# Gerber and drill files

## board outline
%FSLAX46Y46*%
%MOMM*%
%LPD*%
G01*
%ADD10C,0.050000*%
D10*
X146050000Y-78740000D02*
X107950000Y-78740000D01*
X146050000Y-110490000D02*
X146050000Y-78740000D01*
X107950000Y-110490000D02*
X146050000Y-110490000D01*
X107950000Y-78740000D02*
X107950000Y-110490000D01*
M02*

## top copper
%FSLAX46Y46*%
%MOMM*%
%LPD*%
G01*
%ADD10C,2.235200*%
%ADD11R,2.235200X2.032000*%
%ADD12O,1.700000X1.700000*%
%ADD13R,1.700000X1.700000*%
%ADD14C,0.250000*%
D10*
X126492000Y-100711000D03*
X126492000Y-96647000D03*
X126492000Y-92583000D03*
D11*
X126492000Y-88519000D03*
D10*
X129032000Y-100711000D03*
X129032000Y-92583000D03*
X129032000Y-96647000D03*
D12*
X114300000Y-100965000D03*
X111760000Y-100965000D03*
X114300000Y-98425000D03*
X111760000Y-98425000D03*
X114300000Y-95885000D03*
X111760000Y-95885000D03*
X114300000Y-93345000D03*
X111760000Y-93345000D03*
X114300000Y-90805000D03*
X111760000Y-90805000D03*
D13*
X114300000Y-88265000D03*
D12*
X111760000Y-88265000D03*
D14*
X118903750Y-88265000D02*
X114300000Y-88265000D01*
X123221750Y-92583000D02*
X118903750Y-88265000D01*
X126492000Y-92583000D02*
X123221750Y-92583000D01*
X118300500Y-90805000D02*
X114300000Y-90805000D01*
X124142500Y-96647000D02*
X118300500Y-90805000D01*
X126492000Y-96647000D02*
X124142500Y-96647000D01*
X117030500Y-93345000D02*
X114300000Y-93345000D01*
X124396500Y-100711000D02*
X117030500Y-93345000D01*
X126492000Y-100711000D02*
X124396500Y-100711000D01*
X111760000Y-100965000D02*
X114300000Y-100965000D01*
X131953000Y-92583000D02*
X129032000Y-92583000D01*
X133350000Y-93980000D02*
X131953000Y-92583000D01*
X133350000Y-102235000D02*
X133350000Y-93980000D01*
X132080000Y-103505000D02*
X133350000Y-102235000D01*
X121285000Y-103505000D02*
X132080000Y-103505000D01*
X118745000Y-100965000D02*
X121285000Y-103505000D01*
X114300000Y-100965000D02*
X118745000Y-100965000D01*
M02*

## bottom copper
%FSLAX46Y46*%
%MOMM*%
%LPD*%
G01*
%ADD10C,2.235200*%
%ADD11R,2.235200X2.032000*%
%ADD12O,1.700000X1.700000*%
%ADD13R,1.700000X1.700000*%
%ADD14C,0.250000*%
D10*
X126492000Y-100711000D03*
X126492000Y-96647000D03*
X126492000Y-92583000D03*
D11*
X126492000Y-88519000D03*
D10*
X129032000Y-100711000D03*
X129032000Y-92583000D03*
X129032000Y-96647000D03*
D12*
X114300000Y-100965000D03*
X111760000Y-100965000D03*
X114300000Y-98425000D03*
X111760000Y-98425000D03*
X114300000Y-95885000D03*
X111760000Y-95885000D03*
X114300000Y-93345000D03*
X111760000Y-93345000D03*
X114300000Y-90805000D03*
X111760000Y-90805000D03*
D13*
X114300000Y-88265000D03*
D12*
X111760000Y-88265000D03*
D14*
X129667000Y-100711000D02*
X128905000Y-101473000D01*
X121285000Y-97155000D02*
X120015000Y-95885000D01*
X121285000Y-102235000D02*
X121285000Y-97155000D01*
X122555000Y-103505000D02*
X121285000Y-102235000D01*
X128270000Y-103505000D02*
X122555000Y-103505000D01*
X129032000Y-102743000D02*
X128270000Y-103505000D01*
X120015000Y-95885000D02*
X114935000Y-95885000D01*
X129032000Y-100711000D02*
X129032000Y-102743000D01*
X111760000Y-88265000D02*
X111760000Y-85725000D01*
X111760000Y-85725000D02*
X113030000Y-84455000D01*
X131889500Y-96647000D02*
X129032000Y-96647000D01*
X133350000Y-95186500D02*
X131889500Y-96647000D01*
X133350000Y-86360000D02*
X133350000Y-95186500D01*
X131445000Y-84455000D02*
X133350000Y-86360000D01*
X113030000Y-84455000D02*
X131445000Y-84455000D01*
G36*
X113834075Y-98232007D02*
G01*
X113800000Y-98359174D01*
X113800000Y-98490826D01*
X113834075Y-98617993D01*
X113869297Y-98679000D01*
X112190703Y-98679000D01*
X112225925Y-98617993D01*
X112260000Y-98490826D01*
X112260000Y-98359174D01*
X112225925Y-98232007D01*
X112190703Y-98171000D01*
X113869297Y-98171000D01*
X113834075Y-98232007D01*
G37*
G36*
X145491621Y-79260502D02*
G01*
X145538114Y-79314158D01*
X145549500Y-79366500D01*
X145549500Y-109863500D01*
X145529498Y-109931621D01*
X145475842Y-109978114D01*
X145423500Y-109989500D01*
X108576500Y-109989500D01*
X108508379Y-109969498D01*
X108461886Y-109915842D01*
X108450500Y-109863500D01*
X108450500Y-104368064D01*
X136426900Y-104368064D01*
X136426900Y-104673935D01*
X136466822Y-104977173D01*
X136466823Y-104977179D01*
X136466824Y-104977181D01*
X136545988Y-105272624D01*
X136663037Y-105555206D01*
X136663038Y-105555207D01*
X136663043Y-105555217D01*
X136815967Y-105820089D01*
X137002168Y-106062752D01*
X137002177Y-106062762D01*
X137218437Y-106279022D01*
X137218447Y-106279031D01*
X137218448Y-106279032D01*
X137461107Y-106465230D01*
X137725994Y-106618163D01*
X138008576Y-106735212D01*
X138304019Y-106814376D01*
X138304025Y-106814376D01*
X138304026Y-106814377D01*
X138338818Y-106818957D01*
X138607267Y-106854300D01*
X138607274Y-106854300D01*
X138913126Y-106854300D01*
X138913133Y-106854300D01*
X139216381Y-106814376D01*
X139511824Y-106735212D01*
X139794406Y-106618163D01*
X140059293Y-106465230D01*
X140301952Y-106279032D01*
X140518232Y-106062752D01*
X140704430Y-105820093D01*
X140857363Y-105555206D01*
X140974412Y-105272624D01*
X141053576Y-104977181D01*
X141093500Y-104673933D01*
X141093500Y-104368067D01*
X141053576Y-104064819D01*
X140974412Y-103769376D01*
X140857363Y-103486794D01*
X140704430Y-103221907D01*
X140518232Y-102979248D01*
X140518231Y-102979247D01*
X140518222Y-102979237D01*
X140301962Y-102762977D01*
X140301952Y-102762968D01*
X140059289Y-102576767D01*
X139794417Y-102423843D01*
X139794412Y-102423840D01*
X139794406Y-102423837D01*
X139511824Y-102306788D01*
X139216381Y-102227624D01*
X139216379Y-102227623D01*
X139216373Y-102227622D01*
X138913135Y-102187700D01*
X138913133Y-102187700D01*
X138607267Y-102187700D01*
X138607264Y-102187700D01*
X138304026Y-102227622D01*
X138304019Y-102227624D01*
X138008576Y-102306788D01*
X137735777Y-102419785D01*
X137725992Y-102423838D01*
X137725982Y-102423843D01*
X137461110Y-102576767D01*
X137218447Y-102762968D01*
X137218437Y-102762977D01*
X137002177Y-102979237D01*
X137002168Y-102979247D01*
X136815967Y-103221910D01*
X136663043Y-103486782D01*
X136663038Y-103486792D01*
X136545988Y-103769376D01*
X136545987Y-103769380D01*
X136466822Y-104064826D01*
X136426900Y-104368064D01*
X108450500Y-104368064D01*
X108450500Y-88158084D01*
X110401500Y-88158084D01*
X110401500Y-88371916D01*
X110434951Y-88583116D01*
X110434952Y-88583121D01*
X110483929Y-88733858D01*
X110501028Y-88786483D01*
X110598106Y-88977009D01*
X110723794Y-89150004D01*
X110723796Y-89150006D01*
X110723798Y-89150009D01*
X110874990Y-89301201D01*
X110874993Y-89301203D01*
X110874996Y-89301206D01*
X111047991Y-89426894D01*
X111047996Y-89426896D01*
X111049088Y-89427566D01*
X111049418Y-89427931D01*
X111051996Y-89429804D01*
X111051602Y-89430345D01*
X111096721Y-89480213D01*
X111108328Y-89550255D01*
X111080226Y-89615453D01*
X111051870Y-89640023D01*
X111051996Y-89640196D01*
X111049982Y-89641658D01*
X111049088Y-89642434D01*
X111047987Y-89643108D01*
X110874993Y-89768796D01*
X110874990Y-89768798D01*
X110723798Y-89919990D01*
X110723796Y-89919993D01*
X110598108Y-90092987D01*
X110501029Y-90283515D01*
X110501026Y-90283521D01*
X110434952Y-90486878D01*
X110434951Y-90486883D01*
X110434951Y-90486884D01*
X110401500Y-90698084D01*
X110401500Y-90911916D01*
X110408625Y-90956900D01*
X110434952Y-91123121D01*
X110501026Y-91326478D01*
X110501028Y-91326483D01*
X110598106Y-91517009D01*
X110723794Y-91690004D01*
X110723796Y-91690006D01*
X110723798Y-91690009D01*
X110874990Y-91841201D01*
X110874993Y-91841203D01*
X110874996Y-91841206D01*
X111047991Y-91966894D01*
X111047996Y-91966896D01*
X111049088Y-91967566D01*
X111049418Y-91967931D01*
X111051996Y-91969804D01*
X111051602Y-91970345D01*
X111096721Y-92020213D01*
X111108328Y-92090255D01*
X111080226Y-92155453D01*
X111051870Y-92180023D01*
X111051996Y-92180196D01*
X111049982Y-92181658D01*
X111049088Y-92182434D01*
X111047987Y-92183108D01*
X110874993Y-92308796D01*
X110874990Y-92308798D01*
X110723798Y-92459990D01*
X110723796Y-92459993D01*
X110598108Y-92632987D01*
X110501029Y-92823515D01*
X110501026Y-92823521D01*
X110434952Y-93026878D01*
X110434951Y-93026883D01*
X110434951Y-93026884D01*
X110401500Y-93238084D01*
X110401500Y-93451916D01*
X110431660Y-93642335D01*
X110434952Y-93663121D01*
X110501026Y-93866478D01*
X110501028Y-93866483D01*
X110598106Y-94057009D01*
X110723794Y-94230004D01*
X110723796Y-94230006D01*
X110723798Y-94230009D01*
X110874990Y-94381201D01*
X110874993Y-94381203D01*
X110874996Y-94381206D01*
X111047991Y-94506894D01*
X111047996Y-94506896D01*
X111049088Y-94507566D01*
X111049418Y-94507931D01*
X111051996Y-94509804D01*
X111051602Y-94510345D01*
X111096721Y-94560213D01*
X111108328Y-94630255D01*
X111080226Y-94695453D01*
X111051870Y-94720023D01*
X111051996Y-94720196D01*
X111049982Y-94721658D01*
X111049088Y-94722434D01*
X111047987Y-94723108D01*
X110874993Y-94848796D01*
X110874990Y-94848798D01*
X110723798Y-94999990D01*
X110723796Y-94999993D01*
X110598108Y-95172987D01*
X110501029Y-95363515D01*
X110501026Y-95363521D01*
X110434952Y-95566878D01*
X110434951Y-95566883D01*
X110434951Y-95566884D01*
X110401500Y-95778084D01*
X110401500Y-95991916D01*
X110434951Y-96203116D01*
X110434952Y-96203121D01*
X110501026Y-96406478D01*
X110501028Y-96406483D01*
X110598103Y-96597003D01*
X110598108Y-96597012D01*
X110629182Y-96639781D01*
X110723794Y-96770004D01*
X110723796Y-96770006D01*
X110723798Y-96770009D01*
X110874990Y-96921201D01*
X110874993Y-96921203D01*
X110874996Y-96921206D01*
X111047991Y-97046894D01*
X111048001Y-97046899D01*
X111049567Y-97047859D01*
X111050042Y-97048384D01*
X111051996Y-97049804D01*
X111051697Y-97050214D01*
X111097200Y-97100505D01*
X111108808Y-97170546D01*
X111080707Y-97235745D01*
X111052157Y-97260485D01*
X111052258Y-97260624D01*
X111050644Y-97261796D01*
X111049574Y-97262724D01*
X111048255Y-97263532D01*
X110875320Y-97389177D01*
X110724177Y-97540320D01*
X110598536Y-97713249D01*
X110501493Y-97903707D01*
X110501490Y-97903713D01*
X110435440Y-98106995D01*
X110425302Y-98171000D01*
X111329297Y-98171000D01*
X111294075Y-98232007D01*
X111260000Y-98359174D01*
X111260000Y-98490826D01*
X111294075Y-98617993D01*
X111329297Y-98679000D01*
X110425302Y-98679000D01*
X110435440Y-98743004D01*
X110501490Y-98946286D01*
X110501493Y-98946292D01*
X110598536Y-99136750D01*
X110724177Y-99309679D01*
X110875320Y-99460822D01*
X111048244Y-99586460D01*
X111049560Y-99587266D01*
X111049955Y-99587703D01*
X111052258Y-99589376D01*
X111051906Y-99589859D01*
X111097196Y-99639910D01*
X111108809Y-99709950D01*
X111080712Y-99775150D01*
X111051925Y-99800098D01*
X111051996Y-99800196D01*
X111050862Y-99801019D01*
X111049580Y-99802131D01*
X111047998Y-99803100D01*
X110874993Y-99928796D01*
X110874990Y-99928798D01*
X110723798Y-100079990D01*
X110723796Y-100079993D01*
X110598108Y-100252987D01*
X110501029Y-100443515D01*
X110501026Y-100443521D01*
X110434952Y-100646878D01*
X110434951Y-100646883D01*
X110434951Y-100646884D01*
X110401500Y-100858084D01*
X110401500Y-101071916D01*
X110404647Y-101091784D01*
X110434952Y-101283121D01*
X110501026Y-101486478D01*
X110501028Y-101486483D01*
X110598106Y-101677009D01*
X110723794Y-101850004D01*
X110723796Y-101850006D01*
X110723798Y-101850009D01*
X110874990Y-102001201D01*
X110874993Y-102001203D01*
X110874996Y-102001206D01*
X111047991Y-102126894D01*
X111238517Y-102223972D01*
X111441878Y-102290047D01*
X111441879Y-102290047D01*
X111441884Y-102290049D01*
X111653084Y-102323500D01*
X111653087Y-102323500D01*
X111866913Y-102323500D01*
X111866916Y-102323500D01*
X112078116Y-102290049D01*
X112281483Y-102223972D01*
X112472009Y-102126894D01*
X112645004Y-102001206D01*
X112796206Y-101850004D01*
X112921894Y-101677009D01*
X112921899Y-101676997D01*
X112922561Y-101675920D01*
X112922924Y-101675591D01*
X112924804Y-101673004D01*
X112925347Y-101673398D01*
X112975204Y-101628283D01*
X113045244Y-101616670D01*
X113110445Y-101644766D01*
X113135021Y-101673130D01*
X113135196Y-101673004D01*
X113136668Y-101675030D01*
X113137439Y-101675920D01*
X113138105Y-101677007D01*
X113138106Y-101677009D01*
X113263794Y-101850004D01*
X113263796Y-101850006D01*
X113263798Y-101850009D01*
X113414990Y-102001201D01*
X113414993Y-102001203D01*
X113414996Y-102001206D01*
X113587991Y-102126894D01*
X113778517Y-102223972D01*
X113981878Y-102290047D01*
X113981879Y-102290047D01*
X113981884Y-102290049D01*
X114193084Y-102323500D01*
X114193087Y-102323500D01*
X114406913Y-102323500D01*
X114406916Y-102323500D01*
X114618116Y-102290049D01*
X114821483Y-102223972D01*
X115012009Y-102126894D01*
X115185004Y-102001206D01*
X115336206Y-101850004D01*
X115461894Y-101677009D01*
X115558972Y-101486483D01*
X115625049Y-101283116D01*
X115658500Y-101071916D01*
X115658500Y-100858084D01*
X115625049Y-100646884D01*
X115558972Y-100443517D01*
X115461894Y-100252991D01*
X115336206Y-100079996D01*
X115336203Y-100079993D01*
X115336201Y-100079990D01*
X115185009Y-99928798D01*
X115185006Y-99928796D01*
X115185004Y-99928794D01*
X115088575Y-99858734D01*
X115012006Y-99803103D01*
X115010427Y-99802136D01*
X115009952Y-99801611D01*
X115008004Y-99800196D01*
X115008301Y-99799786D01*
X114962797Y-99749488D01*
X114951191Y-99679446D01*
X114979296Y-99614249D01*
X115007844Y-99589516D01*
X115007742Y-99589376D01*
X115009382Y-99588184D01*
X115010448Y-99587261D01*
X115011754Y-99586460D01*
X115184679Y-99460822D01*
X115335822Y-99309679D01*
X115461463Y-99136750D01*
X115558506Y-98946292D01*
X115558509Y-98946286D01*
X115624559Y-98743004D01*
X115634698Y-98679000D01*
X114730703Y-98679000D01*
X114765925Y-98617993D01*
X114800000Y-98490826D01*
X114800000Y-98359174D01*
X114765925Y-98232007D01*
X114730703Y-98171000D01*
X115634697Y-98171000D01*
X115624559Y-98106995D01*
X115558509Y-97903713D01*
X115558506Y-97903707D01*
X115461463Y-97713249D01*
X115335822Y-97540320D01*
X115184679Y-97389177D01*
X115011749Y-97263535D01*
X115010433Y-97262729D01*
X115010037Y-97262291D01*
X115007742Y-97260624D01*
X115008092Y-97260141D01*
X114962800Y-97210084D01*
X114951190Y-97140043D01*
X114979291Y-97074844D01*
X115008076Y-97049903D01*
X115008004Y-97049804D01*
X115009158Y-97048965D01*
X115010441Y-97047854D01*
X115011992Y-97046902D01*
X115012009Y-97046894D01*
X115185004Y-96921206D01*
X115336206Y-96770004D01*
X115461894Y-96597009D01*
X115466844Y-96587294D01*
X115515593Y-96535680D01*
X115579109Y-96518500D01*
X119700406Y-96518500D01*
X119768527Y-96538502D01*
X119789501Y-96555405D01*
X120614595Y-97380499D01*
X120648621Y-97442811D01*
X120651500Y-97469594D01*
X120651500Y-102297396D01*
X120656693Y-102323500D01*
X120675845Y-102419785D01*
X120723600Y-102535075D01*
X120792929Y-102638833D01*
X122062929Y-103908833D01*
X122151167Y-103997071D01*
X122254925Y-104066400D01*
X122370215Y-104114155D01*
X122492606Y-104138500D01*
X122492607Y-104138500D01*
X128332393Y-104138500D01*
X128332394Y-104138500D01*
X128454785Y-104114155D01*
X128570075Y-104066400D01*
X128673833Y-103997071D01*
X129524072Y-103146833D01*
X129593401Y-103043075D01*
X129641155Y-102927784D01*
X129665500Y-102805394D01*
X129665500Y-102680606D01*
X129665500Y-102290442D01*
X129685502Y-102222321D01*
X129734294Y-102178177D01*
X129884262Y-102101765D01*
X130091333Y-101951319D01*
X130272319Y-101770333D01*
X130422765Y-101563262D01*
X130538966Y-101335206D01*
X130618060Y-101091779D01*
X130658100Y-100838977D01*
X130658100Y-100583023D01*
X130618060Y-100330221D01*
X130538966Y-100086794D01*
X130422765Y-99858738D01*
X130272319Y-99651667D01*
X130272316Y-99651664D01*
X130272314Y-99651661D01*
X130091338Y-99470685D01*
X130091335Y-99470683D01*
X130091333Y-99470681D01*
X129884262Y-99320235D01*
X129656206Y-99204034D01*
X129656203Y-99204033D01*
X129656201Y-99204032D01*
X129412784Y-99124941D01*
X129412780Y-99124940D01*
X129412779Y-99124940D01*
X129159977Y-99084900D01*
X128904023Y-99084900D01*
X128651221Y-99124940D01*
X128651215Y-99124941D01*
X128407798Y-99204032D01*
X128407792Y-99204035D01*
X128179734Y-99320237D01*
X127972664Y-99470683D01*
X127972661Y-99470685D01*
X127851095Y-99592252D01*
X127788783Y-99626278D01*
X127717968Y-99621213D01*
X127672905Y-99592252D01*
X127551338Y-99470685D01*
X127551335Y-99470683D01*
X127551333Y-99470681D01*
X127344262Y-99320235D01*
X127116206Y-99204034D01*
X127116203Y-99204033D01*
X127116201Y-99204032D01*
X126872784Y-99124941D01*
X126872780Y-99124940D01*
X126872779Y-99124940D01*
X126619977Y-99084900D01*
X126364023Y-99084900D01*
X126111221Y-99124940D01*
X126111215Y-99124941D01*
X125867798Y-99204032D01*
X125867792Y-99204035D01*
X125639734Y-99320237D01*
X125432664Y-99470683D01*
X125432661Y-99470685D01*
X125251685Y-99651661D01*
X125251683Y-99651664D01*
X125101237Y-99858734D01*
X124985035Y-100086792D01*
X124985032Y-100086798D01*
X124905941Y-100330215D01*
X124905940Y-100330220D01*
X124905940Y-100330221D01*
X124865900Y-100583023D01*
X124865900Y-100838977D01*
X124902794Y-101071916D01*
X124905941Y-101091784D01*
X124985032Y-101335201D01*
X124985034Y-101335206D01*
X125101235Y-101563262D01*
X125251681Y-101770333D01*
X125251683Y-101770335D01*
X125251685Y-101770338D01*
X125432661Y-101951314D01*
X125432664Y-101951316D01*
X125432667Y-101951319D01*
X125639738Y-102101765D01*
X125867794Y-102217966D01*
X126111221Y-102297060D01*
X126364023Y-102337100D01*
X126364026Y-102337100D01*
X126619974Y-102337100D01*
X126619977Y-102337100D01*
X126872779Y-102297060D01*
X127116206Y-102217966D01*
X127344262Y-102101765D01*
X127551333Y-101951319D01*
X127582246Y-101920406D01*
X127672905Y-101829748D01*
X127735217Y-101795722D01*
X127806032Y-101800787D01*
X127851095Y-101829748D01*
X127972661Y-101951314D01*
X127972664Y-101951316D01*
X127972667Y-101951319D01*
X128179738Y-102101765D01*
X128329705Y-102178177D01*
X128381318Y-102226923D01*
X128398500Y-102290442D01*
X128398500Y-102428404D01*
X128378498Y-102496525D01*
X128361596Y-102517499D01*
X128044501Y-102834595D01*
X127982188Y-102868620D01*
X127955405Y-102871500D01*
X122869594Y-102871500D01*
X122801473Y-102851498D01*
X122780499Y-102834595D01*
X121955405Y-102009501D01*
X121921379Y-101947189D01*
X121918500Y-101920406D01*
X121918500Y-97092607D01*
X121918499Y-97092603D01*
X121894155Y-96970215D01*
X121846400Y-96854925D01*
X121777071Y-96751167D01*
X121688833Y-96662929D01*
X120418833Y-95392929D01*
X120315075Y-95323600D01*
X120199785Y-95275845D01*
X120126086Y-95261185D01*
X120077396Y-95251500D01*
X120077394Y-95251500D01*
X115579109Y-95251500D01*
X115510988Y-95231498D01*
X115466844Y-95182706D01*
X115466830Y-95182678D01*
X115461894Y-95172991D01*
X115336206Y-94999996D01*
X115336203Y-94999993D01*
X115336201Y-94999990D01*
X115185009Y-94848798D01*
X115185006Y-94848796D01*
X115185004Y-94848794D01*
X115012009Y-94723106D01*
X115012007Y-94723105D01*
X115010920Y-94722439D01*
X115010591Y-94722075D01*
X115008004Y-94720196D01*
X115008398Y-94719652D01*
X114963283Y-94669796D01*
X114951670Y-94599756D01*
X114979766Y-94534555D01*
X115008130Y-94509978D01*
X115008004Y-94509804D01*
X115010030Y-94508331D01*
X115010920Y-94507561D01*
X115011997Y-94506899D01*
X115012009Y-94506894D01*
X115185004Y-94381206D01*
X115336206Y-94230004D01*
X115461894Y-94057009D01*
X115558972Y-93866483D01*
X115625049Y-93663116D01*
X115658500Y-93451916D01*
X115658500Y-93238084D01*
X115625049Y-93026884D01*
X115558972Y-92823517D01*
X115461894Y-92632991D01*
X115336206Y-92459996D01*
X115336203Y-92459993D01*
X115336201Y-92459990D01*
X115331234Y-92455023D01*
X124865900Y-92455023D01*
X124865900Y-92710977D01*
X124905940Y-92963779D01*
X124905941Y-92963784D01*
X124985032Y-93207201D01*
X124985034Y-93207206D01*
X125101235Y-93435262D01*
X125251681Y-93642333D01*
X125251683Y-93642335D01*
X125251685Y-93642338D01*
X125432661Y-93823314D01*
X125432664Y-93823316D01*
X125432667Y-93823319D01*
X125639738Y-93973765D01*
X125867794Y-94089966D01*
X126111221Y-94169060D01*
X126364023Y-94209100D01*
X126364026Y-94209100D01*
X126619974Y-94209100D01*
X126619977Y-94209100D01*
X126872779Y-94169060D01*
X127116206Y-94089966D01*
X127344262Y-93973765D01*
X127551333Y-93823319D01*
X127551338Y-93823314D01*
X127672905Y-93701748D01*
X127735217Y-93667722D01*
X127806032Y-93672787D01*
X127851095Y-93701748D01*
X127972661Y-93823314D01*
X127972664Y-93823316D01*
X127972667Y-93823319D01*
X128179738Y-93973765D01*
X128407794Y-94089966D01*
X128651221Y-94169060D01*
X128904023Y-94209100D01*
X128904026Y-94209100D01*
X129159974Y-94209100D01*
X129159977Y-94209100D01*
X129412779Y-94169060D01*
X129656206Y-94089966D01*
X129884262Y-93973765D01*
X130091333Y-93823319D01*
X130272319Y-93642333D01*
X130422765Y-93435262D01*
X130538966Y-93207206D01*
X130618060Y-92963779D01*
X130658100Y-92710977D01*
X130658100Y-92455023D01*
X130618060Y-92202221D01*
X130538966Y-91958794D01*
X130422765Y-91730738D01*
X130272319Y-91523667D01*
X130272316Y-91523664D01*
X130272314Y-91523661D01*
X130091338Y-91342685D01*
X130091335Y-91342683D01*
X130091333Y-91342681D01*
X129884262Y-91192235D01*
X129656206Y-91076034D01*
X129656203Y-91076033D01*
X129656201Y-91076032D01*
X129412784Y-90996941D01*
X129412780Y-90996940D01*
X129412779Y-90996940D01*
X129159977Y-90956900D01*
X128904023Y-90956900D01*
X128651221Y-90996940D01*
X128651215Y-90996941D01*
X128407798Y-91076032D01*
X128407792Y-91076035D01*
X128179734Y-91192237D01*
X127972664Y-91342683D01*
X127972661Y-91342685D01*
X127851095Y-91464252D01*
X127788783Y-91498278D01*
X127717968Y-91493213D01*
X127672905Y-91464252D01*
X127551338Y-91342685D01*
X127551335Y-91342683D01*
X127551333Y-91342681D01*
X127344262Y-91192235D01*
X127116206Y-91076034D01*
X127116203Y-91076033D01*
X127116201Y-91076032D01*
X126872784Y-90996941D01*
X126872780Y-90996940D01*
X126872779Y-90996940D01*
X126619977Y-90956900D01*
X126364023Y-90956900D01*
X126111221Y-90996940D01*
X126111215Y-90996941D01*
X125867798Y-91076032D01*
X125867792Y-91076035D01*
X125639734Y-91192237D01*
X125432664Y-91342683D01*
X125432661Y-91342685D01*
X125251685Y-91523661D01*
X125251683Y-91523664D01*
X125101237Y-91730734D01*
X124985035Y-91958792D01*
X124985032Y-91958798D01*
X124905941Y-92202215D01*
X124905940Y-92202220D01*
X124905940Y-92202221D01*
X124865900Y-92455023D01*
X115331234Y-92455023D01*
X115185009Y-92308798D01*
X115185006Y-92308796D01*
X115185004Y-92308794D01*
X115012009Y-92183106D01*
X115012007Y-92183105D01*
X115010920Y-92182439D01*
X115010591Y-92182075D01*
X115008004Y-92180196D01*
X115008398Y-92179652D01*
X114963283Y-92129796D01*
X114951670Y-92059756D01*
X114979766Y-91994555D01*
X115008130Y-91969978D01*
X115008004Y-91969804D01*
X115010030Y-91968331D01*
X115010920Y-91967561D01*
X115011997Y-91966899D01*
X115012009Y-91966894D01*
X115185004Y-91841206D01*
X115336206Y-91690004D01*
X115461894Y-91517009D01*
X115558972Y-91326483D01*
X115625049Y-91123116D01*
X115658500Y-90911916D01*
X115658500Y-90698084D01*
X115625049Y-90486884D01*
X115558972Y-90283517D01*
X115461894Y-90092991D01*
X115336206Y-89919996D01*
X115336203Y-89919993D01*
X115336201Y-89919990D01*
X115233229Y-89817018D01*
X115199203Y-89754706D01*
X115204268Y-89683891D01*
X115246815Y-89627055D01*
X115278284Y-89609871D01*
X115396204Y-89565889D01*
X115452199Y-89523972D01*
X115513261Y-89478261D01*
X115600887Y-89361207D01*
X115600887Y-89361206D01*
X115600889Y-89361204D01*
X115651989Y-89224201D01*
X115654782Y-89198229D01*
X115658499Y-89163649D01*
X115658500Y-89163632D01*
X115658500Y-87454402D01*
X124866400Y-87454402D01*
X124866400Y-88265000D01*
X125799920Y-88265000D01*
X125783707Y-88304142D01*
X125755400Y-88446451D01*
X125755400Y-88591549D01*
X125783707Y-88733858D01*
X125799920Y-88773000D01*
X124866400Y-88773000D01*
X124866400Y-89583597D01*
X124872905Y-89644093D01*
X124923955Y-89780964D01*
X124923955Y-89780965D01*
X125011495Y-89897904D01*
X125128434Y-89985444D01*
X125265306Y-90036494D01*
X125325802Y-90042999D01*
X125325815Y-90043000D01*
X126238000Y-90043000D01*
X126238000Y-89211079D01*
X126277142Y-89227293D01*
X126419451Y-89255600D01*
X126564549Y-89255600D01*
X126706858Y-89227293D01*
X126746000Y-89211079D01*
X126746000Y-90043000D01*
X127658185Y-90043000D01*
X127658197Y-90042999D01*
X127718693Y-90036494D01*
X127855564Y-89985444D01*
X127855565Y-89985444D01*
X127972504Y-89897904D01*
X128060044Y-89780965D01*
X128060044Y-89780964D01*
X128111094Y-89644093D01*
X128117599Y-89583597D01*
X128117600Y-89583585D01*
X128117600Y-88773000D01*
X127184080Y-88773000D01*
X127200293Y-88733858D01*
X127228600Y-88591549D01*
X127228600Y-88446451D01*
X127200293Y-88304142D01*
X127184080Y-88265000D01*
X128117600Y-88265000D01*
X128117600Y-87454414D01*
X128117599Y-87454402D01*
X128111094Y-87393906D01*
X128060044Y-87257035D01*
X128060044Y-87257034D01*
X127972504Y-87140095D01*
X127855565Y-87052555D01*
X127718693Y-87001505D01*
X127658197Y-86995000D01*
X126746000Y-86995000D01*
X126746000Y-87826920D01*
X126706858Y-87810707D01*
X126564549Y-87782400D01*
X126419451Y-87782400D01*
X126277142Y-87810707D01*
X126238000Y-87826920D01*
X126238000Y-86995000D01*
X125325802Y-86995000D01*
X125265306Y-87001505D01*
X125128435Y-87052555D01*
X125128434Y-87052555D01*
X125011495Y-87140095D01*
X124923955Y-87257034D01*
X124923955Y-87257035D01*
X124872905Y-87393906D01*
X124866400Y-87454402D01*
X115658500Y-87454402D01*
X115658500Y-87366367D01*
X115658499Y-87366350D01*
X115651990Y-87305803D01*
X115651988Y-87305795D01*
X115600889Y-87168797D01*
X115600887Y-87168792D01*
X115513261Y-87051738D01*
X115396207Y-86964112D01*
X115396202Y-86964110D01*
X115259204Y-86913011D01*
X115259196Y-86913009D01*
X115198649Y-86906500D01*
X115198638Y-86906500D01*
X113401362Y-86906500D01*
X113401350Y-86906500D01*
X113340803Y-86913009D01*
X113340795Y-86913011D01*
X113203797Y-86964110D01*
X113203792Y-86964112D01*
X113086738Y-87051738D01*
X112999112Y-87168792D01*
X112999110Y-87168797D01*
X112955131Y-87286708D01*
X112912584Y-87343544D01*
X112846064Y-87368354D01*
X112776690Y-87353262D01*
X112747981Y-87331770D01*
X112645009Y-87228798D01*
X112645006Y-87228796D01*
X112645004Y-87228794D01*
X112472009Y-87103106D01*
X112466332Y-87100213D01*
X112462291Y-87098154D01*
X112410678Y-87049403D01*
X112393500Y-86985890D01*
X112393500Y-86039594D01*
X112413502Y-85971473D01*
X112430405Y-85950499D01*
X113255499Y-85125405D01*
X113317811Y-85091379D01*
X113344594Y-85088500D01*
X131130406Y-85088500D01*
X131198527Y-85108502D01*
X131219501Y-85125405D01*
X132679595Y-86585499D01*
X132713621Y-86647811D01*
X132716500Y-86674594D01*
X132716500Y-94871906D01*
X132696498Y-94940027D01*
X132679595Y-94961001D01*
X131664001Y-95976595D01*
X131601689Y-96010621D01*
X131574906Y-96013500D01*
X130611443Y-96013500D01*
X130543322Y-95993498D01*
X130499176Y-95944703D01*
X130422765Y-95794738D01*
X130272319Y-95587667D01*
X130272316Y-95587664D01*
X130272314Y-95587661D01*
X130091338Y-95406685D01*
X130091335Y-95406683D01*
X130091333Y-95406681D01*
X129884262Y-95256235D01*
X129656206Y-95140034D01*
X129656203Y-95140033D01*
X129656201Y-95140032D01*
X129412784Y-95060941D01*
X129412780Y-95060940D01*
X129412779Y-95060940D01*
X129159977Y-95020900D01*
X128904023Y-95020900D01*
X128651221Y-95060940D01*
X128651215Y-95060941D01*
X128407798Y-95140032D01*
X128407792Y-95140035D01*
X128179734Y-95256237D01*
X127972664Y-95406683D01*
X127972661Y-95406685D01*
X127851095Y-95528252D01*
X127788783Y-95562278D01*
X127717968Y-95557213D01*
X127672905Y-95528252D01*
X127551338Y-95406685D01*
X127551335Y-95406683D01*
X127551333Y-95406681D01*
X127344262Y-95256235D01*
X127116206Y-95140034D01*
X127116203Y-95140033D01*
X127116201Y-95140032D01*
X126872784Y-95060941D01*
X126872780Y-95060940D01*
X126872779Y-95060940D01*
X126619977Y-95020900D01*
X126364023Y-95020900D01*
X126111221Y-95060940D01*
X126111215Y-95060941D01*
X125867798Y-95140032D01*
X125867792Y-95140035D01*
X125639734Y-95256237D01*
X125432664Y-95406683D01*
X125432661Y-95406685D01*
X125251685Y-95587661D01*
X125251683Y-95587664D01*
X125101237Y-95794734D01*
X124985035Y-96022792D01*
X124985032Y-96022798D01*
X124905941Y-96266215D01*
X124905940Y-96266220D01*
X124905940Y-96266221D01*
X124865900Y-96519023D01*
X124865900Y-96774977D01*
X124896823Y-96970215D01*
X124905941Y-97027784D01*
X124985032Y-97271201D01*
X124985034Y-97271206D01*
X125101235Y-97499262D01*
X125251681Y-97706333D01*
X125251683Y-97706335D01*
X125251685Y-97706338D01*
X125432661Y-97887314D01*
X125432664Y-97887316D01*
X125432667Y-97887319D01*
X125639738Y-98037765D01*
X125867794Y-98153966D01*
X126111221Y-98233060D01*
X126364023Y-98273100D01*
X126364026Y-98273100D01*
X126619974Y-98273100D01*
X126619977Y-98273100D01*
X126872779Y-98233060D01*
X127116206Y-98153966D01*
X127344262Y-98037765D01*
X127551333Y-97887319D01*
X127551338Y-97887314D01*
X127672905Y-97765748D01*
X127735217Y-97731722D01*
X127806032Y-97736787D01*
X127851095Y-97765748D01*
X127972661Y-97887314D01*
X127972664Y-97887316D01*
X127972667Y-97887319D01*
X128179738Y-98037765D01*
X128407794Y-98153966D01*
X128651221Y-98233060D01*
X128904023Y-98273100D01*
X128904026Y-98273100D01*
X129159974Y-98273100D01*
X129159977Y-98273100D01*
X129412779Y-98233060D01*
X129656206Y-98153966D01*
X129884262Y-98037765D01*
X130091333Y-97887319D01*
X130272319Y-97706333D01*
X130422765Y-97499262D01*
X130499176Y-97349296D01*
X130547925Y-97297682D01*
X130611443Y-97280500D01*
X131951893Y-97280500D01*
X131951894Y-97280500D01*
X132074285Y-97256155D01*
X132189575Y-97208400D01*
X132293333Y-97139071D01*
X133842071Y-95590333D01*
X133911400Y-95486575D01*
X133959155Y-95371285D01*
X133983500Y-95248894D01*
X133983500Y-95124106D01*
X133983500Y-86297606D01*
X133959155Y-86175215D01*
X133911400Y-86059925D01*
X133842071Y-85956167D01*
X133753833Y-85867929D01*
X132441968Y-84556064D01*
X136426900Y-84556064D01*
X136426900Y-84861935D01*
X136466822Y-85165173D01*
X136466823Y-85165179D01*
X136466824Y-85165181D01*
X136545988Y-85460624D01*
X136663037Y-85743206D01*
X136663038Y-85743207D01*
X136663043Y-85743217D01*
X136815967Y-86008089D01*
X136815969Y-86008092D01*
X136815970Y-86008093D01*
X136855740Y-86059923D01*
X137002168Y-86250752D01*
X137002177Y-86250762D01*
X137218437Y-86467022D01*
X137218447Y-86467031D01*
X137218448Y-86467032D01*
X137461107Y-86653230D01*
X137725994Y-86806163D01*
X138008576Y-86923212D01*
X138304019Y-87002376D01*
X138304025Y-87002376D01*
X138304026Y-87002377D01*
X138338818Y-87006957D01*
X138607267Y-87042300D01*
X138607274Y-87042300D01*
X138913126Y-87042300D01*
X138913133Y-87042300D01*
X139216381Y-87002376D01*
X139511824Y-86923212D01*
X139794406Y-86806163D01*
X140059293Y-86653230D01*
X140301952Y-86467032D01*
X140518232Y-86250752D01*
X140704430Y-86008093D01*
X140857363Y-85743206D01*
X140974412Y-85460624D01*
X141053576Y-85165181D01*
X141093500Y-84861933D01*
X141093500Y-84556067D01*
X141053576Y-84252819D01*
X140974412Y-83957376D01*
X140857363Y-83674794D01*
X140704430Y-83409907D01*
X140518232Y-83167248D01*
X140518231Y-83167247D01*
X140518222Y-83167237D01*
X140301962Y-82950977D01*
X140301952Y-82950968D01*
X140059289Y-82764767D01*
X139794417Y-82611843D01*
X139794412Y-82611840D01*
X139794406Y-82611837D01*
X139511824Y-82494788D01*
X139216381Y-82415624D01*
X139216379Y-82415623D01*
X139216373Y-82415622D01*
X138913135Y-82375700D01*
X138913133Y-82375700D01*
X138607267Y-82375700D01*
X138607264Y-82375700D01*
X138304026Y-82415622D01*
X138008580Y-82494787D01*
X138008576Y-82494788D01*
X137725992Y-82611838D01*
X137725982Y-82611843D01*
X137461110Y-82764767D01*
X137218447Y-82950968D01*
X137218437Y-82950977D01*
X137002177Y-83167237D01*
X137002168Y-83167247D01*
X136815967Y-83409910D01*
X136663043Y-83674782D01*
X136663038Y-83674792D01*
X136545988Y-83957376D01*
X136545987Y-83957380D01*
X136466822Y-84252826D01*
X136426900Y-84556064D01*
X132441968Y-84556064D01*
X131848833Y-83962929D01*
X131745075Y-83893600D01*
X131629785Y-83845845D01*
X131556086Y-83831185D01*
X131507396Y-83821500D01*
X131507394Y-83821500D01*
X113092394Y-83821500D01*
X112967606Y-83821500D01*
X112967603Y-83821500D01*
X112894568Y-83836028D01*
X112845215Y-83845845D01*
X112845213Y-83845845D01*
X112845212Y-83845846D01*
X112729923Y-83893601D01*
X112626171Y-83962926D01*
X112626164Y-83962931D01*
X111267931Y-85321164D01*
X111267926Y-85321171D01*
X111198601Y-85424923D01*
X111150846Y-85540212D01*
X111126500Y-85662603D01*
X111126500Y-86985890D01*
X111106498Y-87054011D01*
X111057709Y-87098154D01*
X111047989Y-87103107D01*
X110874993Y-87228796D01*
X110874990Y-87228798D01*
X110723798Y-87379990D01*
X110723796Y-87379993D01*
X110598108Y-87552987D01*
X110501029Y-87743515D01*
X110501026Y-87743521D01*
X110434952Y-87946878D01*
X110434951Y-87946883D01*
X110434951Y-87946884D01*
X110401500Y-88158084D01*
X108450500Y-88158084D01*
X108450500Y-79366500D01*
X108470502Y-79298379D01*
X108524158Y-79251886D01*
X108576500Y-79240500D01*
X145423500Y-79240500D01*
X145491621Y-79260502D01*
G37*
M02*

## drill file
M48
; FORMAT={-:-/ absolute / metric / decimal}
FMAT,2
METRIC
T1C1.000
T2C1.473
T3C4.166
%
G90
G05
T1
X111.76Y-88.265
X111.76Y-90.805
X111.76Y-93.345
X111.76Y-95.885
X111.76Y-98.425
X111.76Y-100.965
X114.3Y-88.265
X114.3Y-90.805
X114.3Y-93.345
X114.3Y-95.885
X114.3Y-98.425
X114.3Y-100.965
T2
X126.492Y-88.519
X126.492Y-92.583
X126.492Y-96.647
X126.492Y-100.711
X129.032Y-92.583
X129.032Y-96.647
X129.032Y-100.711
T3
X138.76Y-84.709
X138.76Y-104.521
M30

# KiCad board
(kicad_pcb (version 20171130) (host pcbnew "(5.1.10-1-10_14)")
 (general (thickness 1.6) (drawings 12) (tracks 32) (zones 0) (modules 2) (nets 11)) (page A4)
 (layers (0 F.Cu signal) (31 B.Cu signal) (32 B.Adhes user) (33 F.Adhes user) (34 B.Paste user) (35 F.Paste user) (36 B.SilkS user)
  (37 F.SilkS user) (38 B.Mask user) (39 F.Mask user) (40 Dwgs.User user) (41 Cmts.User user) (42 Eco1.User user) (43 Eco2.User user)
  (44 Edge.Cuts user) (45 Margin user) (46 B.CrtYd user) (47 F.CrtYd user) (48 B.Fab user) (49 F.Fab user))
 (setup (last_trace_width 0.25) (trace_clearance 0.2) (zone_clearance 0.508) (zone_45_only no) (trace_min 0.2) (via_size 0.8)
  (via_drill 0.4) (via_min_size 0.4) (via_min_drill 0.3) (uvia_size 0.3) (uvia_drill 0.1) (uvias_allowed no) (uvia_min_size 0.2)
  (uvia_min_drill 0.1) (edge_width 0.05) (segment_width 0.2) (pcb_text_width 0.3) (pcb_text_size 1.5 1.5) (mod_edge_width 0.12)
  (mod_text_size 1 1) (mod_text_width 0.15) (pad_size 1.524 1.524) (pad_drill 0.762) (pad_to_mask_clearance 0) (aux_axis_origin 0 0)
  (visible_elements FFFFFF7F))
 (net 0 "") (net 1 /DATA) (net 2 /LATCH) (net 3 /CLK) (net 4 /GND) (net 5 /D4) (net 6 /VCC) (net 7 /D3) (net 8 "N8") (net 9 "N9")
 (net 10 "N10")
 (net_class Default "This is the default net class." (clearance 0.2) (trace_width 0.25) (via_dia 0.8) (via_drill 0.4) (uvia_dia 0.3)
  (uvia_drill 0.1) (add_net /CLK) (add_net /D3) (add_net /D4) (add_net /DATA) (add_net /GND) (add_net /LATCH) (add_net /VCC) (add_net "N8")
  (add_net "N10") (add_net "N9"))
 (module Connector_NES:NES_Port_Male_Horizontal (layer F.Cu) (at 125.73 94.615 180)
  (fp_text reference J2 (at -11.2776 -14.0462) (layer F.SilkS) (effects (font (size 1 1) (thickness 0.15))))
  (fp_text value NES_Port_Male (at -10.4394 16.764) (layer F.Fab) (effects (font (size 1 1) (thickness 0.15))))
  (pad 4 thru_hole circle (at -0.762 -6.096 180) (size 2.2352 2.2352) (drill 1.4732) (layers *.Cu *.Mask) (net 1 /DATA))
  (pad 3 thru_hole circle (at -0.762 -2.032 180) (size 2.2352 2.2352) (drill 1.4732) (layers *.Cu *.Mask) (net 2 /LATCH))
  (pad 2 thru_hole circle (at -0.762 2.032 180) (size 2.2352 2.2352) (drill 1.4732) (layers *.Cu *.Mask) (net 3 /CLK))
  (pad 1 thru_hole rect (at -0.762 6.096 180) (size 2.2352 2.032) (drill 1.4732) (layers *.Cu *.Mask) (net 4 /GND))
  (pad 5 thru_hole circle (at -3.302 -6.096 180) (size 2.2352 2.2352) (drill 1.4732) (layers *.Cu *.Mask) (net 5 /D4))
  (pad 7 thru_hole circle (at -3.302 2.032 180) (size 2.2352 2.2352) (drill 1.4732) (layers *.Cu *.Mask) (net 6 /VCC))
  (pad 6 thru_hole circle (at -3.302 -2.032 180) (size 2.2352 2.2352) (drill 1.4732) (layers *.Cu *.Mask) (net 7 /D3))
  (pad "" np_thru_hole circle (at -13.0302 -9.906 180) (size 4.1656 4.1656) (drill 4.1656) (layers *.Cu *.Mask))
  (pad "" np_thru_hole circle (at -13.0302 9.906 180) (size 4.1656 4.1656) (drill 4.1656) (layers *.Cu *.Mask)))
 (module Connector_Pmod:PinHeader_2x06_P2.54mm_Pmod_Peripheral (layer F.Cu) (at 114.3 100.965)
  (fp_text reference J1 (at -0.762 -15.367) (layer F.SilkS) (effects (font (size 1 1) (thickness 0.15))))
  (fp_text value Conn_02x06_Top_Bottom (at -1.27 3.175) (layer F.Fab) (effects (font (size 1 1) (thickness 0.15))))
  (pad 6 thru_hole oval (at 0 0 180) (size 1.7 1.7) (drill 1) (layers *.Cu *.Mask) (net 6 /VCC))
  (pad 12 thru_hole oval (at -2.54 0 180) (size 1.7 1.7) (drill 1) (layers *.Cu *.Mask) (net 6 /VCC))
  (pad 5 thru_hole oval (at 0 -2.54 180) (size 1.7 1.7) (drill 1) (layers *.Cu *.Mask) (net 4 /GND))
  (pad 11 thru_hole oval (at -2.54 -2.54 180) (size 1.7 1.7) (drill 1) (layers *.Cu *.Mask) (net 4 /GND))
  (pad 4 thru_hole oval (at 0 -5.08 180) (size 1.7 1.7) (drill 1) (layers *.Cu *.Mask) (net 5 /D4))
  (pad 10 thru_hole oval (at -2.54 -5.08 180) (size 1.7 1.7) (drill 1) (layers *.Cu *.Mask) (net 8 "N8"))
  (pad 3 thru_hole oval (at 0 -7.62 180) (size 1.7 1.7) (drill 1) (layers *.Cu *.Mask) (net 1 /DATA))
  (pad 9 thru_hole oval (at -2.54 -7.62 180) (size 1.7 1.7) (drill 1) (layers *.Cu *.Mask) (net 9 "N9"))
  (pad 2 thru_hole oval (at 0 -10.16 180) (size 1.7 1.7) (drill 1) (layers *.Cu *.Mask) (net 2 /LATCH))
  (pad 8 thru_hole oval (at -2.54 -10.16 180) (size 1.7 1.7) (drill 1) (layers *.Cu *.Mask) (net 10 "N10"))
  (pad 1 thru_hole rect (at 0 -12.7 180) (size 1.7 1.7) (drill 1) (layers *.Cu *.Mask) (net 3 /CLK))
  (pad 7 thru_hole oval (at -2.54 -12.7 180) (size 1.7 1.7) (drill 1) (layers *.Cu *.Mask) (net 7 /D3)))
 (gr_line (start 146.05 78.74) (end 107.95 78.74) (layer Edge.Cuts) (width 0.05))
 (gr_line (start 146.05 110.49) (end 146.05 78.74) (layer Edge.Cuts) (width 0.05))
 (gr_line (start 107.95 110.49) (end 146.05 110.49) (layer Edge.Cuts) (width 0.05))
 (gr_line (start 107.95 78.74) (end 107.95 110.49) (layer Edge.Cuts) (width 0.05))
 (segment (start 118.90375 88.265) (end 114.3 88.265) (width 0.25) (layer F.Cu) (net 3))
 (segment (start 123.22175 92.583) (end 118.90375 88.265) (width 0.25) (layer F.Cu) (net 3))
 (segment (start 126.492 92.583) (end 123.22175 92.583) (width 0.25) (layer F.Cu) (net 3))
 (segment (start 118.3005 90.805) (end 114.3 90.805) (width 0.25) (layer F.Cu) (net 2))
 (segment (start 124.1425 96.647) (end 118.3005 90.805) (width 0.25) (layer F.Cu) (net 2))
 (segment (start 126.492 96.647) (end 124.1425 96.647) (width 0.25) (layer F.Cu) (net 2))
 (segment (start 117.0305 93.345) (end 114.3 93.345) (width 0.25) (layer F.Cu) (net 1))
 (segment (start 124.3965 100.711) (end 117.0305 93.345) (width 0.25) (layer F.Cu) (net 1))
 (segment (start 126.492 100.711) (end 124.3965 100.711) (width 0.25) (layer F.Cu) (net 1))
 (segment (start 129.667 100.711) (end 128.905 101.473) (width 0.25) (layer B.Cu) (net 5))
 (segment (start 121.285 97.155) (end 120.015 95.885) (width 0.25) (layer B.Cu) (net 5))
 (segment (start 121.285 102.235) (end 121.285 97.155) (width 0.25) (layer B.Cu) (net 5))
 (segment (start 122.555 103.505) (end 121.285 102.235) (width 0.25) (layer B.Cu) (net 5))
 (segment (start 128.27 103.505) (end 122.555 103.505) (width 0.25) (layer B.Cu) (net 5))
 (segment (start 129.032 102.743) (end 128.27 103.505) (width 0.25) (layer B.Cu) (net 5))
 (segment (start 120.015 95.885) (end 114.935 95.885) (width 0.25) (layer B.Cu) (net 5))
 (segment (start 129.032 100.711) (end 129.032 102.743) (width 0.25) (layer B.Cu) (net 5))
 (segment (start 111.76 100.965) (end 114.3 100.965) (width 0.25) (layer F.Cu) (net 6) (status 30))
 (segment (start 131.953 92.583) (end 129.032 92.583) (width 0.25) (layer F.Cu) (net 6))
 (segment (start 133.35 93.98) (end 131.953 92.583) (width 0.25) (layer F.Cu) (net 6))
 (segment (start 133.35 102.235) (end 133.35 93.98) (width 0.25) (layer F.Cu) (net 6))
 (segment (start 132.08 103.505) (end 133.35 102.235) (width 0.25) (layer F.Cu) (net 6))
 (segment (start 121.285 103.505) (end 132.08 103.505) (width 0.25) (layer F.Cu) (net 6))
 (segment (start 118.745 100.965) (end 121.285 103.505) (width 0.25) (layer F.Cu) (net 6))
 (segment (start 114.3 100.965) (end 118.745 100.965) (width 0.25) (layer F.Cu) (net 6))
 (segment (start 111.76 88.265) (end 111.76 85.725) (width 0.25) (layer B.Cu) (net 7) (status 10))
 (segment (start 111.76 85.725) (end 113.03 84.455) (width 0.25) (layer B.Cu) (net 7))
 (segment (start 131.8895 96.647) (end 129.032 96.647) (width 0.25) (layer B.Cu) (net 7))
 (segment (start 133.35 95.1865) (end 131.8895 96.647) (width 0.25) (layer B.Cu) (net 7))
 (segment (start 133.35 86.36) (end 133.35 95.1865) (width 0.25) (layer B.Cu) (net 7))
 (segment (start 131.445 84.455) (end 133.35 86.36) (width 0.25) (layer B.Cu) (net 7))
 (segment (start 113.03 84.455) (end 131.445 84.455) (width 0.25) (layer B.Cu) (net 7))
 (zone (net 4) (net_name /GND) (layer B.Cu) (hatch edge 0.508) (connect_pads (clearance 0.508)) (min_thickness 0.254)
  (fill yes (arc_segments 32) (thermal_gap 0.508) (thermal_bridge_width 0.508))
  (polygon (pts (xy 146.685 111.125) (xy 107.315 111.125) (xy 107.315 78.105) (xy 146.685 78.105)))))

